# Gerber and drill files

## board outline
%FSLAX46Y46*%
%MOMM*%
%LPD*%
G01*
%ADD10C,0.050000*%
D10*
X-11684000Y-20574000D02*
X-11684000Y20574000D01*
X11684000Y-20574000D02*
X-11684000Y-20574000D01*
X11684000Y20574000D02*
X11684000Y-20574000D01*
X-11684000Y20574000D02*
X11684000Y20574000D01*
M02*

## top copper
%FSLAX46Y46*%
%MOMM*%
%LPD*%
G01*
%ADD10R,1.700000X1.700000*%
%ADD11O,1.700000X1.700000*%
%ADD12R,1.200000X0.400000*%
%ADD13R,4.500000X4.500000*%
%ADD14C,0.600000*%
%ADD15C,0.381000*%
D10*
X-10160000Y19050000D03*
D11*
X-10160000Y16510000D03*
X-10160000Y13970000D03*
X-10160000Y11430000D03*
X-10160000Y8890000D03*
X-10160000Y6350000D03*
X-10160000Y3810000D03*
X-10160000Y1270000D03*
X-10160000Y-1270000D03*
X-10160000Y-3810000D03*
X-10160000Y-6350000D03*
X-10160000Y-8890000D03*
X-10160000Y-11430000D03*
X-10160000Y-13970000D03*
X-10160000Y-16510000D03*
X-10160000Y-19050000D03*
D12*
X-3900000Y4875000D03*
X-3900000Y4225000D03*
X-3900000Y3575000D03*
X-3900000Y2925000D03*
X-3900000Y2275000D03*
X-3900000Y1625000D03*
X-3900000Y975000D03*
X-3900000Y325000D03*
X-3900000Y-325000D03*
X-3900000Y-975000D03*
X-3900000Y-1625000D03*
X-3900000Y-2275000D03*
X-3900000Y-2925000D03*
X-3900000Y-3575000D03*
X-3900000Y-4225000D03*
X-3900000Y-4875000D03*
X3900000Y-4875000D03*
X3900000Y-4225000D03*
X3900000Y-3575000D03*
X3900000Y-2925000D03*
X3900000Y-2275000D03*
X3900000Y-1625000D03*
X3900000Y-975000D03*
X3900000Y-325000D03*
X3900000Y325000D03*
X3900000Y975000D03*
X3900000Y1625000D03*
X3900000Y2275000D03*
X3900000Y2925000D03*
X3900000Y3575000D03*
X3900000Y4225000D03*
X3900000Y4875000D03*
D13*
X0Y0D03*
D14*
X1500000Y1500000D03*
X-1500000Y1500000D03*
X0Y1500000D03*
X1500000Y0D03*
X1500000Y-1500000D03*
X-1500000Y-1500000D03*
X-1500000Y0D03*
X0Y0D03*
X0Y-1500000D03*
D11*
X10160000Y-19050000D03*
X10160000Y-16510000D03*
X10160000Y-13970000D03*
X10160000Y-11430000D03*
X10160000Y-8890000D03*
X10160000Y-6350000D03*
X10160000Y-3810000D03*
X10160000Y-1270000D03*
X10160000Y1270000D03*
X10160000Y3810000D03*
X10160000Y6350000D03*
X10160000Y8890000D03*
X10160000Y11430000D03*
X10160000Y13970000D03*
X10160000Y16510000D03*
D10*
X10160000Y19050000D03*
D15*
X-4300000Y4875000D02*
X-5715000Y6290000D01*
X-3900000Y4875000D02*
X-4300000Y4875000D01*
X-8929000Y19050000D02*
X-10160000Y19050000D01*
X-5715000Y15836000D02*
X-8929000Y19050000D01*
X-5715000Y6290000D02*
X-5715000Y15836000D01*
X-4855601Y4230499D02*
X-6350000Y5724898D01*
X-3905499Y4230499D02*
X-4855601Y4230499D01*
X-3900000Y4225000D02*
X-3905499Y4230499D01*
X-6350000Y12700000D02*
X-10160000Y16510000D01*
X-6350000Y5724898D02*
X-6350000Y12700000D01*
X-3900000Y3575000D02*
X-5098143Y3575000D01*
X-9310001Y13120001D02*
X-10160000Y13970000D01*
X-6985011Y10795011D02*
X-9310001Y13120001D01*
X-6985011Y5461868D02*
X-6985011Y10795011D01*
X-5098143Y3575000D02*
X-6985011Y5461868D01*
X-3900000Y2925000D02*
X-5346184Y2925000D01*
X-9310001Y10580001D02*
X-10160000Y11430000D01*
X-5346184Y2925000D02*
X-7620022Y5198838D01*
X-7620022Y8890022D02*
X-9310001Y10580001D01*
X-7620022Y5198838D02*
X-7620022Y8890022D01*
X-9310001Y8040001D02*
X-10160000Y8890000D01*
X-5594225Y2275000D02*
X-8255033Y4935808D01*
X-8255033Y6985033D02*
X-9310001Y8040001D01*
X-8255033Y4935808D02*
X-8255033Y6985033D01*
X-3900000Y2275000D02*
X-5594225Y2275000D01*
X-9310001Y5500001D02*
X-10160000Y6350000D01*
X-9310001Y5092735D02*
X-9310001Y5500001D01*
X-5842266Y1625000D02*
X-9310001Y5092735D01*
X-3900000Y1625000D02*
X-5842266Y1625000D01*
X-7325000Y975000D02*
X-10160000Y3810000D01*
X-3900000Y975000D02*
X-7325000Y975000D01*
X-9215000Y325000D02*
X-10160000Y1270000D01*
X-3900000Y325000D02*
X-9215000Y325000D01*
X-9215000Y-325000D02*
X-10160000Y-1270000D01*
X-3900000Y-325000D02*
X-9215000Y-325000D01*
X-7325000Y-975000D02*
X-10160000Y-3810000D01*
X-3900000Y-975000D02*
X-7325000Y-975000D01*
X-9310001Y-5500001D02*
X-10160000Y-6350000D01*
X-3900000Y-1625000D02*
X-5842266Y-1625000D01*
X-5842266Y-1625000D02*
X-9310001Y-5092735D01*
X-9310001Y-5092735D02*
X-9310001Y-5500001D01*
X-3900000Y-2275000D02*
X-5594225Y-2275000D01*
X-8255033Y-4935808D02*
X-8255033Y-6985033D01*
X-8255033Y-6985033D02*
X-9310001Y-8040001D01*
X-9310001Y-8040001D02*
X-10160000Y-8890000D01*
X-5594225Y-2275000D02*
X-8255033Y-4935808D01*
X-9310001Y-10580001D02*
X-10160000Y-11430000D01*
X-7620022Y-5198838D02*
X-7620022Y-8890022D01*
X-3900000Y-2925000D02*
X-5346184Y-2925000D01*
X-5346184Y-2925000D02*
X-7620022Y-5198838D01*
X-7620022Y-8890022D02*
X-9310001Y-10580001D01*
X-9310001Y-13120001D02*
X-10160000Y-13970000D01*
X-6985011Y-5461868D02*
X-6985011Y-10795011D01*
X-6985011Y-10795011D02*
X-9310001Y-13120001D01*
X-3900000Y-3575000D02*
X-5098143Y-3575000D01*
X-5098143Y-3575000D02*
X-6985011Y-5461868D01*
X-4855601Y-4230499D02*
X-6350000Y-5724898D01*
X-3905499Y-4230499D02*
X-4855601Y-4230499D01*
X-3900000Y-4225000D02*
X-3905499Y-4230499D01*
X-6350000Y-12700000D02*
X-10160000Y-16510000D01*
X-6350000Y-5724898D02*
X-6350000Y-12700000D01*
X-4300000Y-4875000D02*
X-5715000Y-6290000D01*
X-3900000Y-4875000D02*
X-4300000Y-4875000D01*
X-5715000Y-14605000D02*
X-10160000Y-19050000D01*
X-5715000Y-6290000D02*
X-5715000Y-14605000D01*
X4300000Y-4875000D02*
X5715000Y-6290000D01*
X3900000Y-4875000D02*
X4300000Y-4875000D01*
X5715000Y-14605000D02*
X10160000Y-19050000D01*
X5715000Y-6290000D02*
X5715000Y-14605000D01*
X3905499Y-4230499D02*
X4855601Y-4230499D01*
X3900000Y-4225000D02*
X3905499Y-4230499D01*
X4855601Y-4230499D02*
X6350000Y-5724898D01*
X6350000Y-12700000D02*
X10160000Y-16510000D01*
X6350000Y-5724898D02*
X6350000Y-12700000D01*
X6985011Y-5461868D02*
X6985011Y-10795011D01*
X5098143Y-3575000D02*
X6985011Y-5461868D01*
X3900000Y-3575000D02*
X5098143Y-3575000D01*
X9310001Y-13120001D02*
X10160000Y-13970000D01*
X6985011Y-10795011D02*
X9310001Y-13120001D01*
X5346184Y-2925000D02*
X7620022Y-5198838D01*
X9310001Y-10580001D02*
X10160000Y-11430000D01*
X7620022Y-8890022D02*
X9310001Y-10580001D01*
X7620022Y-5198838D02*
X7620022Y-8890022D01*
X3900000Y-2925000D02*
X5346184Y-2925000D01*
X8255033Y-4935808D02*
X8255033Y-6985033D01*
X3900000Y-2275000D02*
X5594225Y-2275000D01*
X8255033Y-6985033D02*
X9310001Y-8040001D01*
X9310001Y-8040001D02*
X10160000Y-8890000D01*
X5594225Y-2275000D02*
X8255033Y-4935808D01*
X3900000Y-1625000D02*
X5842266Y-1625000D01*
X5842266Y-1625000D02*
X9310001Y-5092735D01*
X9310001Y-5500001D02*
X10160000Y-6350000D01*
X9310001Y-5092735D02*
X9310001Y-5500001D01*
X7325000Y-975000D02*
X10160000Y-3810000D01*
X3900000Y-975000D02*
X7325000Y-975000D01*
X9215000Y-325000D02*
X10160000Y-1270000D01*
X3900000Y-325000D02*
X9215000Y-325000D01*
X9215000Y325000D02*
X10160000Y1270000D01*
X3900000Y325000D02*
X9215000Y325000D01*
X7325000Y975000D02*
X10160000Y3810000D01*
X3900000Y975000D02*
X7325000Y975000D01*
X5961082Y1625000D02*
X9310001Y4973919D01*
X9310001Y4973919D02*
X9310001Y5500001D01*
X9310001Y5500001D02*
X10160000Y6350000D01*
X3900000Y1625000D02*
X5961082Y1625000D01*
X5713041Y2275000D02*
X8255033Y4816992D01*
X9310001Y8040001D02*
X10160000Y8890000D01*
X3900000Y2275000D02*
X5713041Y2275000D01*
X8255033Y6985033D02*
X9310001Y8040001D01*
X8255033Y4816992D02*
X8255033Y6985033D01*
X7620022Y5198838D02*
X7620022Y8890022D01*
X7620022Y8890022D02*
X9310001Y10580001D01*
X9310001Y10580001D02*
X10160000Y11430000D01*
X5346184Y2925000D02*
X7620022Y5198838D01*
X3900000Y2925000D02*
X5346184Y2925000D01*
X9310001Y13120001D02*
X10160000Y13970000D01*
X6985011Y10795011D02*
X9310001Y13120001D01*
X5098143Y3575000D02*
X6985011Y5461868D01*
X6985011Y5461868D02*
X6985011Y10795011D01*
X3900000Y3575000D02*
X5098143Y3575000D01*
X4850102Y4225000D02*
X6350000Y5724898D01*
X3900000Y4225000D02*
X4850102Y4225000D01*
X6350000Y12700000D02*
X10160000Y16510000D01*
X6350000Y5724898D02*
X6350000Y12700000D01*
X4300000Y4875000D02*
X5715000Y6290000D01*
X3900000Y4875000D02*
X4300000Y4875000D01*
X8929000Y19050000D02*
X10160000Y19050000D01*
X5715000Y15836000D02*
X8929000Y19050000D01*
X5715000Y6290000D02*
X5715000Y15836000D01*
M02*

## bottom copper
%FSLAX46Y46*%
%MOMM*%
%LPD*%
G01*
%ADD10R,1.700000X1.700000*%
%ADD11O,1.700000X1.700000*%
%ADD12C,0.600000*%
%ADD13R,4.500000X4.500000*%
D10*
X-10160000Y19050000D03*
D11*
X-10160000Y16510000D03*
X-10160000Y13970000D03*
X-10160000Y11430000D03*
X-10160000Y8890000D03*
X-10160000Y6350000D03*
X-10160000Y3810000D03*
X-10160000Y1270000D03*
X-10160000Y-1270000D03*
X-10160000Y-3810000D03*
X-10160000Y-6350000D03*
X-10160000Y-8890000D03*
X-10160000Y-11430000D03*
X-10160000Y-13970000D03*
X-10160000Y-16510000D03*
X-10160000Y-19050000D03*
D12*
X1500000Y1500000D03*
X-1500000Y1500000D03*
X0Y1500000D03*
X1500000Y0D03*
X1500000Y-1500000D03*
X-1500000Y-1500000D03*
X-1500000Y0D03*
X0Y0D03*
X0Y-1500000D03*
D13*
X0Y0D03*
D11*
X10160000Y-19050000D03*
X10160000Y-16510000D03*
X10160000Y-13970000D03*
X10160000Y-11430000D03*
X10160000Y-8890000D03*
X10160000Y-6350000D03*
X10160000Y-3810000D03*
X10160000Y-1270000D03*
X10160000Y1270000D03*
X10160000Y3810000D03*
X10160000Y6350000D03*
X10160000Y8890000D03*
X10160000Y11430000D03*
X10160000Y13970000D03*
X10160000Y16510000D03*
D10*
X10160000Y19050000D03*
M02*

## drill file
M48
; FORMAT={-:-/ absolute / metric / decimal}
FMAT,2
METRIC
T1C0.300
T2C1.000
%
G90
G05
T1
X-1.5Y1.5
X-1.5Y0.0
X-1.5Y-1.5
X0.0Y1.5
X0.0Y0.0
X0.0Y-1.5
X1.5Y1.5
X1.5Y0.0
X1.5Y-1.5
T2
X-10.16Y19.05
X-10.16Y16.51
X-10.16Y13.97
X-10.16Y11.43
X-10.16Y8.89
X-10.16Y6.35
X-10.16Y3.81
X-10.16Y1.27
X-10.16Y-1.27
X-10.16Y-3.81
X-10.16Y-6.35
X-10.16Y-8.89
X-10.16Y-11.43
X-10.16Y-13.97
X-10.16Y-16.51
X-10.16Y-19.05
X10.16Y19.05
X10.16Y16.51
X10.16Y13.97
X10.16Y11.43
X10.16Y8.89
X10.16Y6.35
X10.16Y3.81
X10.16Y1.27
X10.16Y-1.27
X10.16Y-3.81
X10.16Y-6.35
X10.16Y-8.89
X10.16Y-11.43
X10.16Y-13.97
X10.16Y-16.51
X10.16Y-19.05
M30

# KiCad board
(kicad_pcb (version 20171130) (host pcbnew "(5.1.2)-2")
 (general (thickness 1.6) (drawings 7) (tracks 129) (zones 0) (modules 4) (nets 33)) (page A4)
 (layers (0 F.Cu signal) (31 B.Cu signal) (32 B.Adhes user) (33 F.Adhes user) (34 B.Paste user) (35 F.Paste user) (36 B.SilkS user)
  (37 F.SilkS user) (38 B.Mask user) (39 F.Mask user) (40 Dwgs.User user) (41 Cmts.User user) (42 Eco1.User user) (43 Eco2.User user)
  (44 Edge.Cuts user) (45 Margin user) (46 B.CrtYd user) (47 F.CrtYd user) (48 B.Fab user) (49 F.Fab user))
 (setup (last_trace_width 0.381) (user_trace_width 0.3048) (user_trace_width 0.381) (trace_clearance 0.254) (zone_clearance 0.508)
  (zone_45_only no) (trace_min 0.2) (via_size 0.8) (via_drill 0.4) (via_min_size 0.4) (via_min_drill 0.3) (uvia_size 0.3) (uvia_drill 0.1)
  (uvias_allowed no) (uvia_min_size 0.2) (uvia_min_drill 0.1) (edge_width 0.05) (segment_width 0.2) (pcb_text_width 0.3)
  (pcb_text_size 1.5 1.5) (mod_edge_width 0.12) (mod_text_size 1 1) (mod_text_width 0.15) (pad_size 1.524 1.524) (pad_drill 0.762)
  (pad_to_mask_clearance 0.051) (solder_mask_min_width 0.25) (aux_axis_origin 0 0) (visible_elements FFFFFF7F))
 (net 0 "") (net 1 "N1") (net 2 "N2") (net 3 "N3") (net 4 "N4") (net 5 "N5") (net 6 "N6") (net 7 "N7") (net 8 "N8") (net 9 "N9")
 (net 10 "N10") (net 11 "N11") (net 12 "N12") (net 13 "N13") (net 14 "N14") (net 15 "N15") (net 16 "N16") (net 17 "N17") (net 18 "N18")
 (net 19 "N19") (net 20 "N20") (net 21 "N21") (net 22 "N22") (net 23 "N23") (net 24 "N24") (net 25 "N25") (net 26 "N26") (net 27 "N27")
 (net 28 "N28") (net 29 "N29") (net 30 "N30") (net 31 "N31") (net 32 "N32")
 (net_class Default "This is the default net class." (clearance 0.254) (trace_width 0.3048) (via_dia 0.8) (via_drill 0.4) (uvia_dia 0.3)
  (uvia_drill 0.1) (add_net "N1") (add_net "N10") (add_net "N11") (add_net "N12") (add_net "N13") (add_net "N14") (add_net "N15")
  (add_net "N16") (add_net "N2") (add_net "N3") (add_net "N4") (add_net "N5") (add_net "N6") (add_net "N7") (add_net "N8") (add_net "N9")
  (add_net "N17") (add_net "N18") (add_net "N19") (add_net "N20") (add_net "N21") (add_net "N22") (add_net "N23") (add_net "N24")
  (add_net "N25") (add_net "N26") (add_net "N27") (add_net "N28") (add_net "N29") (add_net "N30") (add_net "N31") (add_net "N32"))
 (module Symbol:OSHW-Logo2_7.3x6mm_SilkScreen (layer F.Cu) (at 0 10.668)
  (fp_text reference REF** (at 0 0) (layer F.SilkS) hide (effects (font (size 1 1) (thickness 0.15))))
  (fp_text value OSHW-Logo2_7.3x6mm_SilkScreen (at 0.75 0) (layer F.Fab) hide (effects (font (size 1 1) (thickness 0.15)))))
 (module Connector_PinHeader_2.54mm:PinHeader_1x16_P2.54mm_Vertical (layer B.Cu) (at -10.16 -19.05 180)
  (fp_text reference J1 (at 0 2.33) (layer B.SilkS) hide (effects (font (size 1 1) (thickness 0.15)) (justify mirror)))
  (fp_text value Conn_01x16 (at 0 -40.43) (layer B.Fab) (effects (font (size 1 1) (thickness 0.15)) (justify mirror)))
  (pad 1 thru_hole rect (at 0 0 180) (size 1.7 1.7) (drill 1) (layers *.Cu *.Mask) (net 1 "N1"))
  (pad 2 thru_hole oval (at 0 -2.54 180) (size 1.7 1.7) (drill 1) (layers *.Cu *.Mask) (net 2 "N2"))
  (pad 3 thru_hole oval (at 0 -5.08 180) (size 1.7 1.7) (drill 1) (layers *.Cu *.Mask) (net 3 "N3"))
  (pad 4 thru_hole oval (at 0 -7.62 180) (size 1.7 1.7) (drill 1) (layers *.Cu *.Mask) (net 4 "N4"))
  (pad 5 thru_hole oval (at 0 -10.16 180) (size 1.7 1.7) (drill 1) (layers *.Cu *.Mask) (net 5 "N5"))
  (pad 6 thru_hole oval (at 0 -12.7 180) (size 1.7 1.7) (drill 1) (layers *.Cu *.Mask) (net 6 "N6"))
  (pad 7 thru_hole oval (at 0 -15.24 180) (size 1.7 1.7) (drill 1) (layers *.Cu *.Mask) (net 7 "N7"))
  (pad 8 thru_hole oval (at 0 -17.78 180) (size 1.7 1.7) (drill 1) (layers *.Cu *.Mask) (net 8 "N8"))
  (pad 9 thru_hole oval (at 0 -20.32 180) (size 1.7 1.7) (drill 1) (layers *.Cu *.Mask) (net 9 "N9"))
  (pad 10 thru_hole oval (at 0 -22.86 180) (size 1.7 1.7) (drill 1) (layers *.Cu *.Mask) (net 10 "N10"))
  (pad 11 thru_hole oval (at 0 -25.4 180) (size 1.7 1.7) (drill 1) (layers *.Cu *.Mask) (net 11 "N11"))
  (pad 12 thru_hole oval (at 0 -27.94 180) (size 1.7 1.7) (drill 1) (layers *.Cu *.Mask) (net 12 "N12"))
  (pad 13 thru_hole oval (at 0 -30.48 180) (size 1.7 1.7) (drill 1) (layers *.Cu *.Mask) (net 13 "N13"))
  (pad 14 thru_hole oval (at 0 -33.02 180) (size 1.7 1.7) (drill 1) (layers *.Cu *.Mask) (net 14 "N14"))
  (pad 15 thru_hole oval (at 0 -35.56 180) (size 1.7 1.7) (drill 1) (layers *.Cu *.Mask) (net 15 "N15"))
  (pad 16 thru_hole oval (at 0 -38.1 180) (size 1.7 1.7) (drill 1) (layers *.Cu *.Mask) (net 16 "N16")))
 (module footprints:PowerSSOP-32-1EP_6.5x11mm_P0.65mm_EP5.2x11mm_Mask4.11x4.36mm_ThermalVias (layer F.Cu) (at 0 0)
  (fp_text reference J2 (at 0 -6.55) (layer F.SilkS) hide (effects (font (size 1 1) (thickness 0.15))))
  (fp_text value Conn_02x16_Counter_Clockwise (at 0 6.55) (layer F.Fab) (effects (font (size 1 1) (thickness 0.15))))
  (pad 1 smd rect (at -3.9 -4.875) (size 1.2 0.4) (layers F.Cu F.Paste F.Mask) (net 1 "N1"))
  (pad 2 smd rect (at -3.9 -4.225) (size 1.2 0.4) (layers F.Cu F.Paste F.Mask) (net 2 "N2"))
  (pad 3 smd rect (at -3.9 -3.575) (size 1.2 0.4) (layers F.Cu F.Paste F.Mask) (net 3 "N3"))
  (pad 4 smd rect (at -3.9 -2.925) (size 1.2 0.4) (layers F.Cu F.Paste F.Mask) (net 4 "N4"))
  (pad 5 smd rect (at -3.9 -2.275) (size 1.2 0.4) (layers F.Cu F.Paste F.Mask) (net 5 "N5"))
  (pad 6 smd rect (at -3.9 -1.625) (size 1.2 0.4) (layers F.Cu F.Paste F.Mask) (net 6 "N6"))
  (pad 7 smd rect (at -3.9 -0.975) (size 1.2 0.4) (layers F.Cu F.Paste F.Mask) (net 7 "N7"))
  (pad 8 smd rect (at -3.9 -0.325) (size 1.2 0.4) (layers F.Cu F.Paste F.Mask) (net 8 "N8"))
  (pad 9 smd rect (at -3.9 0.325) (size 1.2 0.4) (layers F.Cu F.Paste F.Mask) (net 9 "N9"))
  (pad 10 smd rect (at -3.9 0.975) (size 1.2 0.4) (layers F.Cu F.Paste F.Mask) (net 10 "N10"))
  (pad 11 smd rect (at -3.9 1.625) (size 1.2 0.4) (layers F.Cu F.Paste F.Mask) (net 11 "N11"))
  (pad 12 smd rect (at -3.9 2.275) (size 1.2 0.4) (layers F.Cu F.Paste F.Mask) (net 12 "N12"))
  (pad 13 smd rect (at -3.9 2.925) (size 1.2 0.4) (layers F.Cu F.Paste F.Mask) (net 13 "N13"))
  (pad 14 smd rect (at -3.9 3.575) (size 1.2 0.4) (layers F.Cu F.Paste F.Mask) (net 14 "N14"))
  (pad 15 smd rect (at -3.9 4.225) (size 1.2 0.4) (layers F.Cu F.Paste F.Mask) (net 15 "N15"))
  (pad 16 smd rect (at -3.9 4.875) (size 1.2 0.4) (layers F.Cu F.Paste F.Mask) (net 16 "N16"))
  (pad 17 smd rect (at 3.9 4.875) (size 1.2 0.4) (layers F.Cu F.Paste F.Mask) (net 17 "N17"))
  (pad 18 smd rect (at 3.9 4.225) (size 1.2 0.4) (layers F.Cu F.Paste F.Mask) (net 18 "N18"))
  (pad 19 smd rect (at 3.9 3.575) (size 1.2 0.4) (layers F.Cu F.Paste F.Mask) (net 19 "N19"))
  (pad 20 smd rect (at 3.9 2.925) (size 1.2 0.4) (layers F.Cu F.Paste F.Mask) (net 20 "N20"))
  (pad 21 smd rect (at 3.9 2.275) (size 1.2 0.4) (layers F.Cu F.Paste F.Mask) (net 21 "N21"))
  (pad 22 smd rect (at 3.9 1.625) (size 1.2 0.4) (layers F.Cu F.Paste F.Mask) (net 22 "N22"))
  (pad 23 smd rect (at 3.9 0.975) (size 1.2 0.4) (layers F.Cu F.Paste F.Mask) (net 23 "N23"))
  (pad 24 smd rect (at 3.9 0.325) (size 1.2 0.4) (layers F.Cu F.Paste F.Mask) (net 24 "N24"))
  (pad 25 smd rect (at 3.9 -0.325) (size 1.2 0.4) (layers F.Cu F.Paste F.Mask) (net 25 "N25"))
  (pad 26 smd rect (at 3.9 -0.975) (size 1.2 0.4) (layers F.Cu F.Paste F.Mask) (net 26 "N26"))
  (pad 27 smd rect (at 3.9 -1.625) (size 1.2 0.4) (layers F.Cu F.Paste F.Mask) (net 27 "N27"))
  (pad 28 smd rect (at 3.9 -2.275) (size 1.2 0.4) (layers F.Cu F.Paste F.Mask) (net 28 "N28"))
  (pad 29 smd rect (at 3.9 -2.925) (size 1.2 0.4) (layers F.Cu F.Paste F.Mask) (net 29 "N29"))
  (pad 30 smd rect (at 3.9 -3.575) (size 1.2 0.4) (layers F.Cu F.Paste F.Mask) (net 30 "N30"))
  (pad 31 smd rect (at 3.9 -4.225) (size 1.2 0.4) (layers F.Cu F.Paste F.Mask) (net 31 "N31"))
  (pad 32 smd rect (at 3.9 -4.875) (size 1.2 0.4) (layers F.Cu F.Paste F.Mask) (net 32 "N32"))
  (pad 33 smd rect (at 0 0) (size 4.5 4.5) (layers F.Cu)) (pad "" smd rect (at 0 0) (size 4.11 4.36) (layers F.Mask))
  (pad 33 thru_hole circle (at 1.5 -1.5) (size 0.6 0.6) (drill 0.3) (layers *.Cu))
  (pad 33 thru_hole circle (at -1.5 -1.5) (size 0.6 0.6) (drill 0.3) (layers *.Cu))
  (pad 33 thru_hole circle (at 0 -1.5) (size 0.6 0.6) (drill 0.3) (layers *.Cu))
  (pad 33 thru_hole circle (at 1.5 0) (size 0.6 0.6) (drill 0.3) (layers *.Cu))
  (pad 33 thru_hole circle (at 1.5 1.5) (size 0.6 0.6) (drill 0.3) (layers *.Cu))
  (pad 33 thru_hole circle (at -1.5 1.5) (size 0.6 0.6) (drill 0.3) (layers *.Cu))
  (pad 33 thru_hole circle (at -1.5 0) (size 0.6 0.6) (drill 0.3) (layers *.Cu))
  (pad 33 thru_hole circle (at 0 0) (size 0.6 0.6) (drill 0.3) (layers *.Cu))
  (pad 33 thru_hole circle (at 0 1.5) (size 0.6 0.6) (drill 0.3) (layers *.Cu)) (pad "" smd rect (at 0 -0.65) (size 1.2 1) (layers F.Paste))
  (pad "" smd rect (at 0 0.65) (size 1.2 1) (layers F.Paste))
  (pad "" smd rect (at 0 1.725) (size 1.2 0.55) (layers F.Paste))
  (pad "" smd rect (at 0 -1.725) (size 1.2 0.55) (layers F.Paste))
  (pad "" smd rect (at -1.365 -0.65) (size 0.93 1) (layers F.Paste))
  (pad "" smd rect (at -1.365 0.65) (size 0.93 1) (layers F.Paste))
  (pad "" smd rect (at 1.365 0.65) (size 0.93 1) (layers F.Paste))
  (pad "" smd rect (at 1.365 -0.65) (size 0.93 1) (layers F.Paste))
  (pad "" smd rect (at 1.365 -1.725) (size 0.93 0.55) (layers F.Paste))
  (pad "" smd rect (at 1.365 1.725) (size 0.93 0.55) (layers F.Paste))
  (pad "" smd rect (at -1.365 1.725) (size 0.93 0.55) (layers F.Paste))
  (pad "" smd rect (at -1.365 -1.725) (size 0.93 0.55) (layers F.Paste)) (pad 33 smd rect (at 0 0) (size 4.5 4.5) (layers B.Cu))
  (pad "" smd rect (at 0 0) (size 4.11 4.36) (layers B.Mask)))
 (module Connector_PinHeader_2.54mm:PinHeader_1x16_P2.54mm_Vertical (layer B.Cu) (at 10.16 -19.05 180)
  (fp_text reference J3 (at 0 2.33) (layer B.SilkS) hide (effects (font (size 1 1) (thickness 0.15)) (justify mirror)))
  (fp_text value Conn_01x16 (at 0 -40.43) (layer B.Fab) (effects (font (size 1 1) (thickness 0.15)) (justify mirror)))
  (pad 16 thru_hole oval (at 0 -38.1 180) (size 1.7 1.7) (drill 1) (layers *.Cu *.Mask) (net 17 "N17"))
  (pad 15 thru_hole oval (at 0 -35.56 180) (size 1.7 1.7) (drill 1) (layers *.Cu *.Mask) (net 18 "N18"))
  (pad 14 thru_hole oval (at 0 -33.02 180) (size 1.7 1.7) (drill 1) (layers *.Cu *.Mask) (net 19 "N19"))
  (pad 13 thru_hole oval (at 0 -30.48 180) (size 1.7 1.7) (drill 1) (layers *.Cu *.Mask) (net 20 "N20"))
  (pad 12 thru_hole oval (at 0 -27.94 180) (size 1.7 1.7) (drill 1) (layers *.Cu *.Mask) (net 21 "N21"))
  (pad 11 thru_hole oval (at 0 -25.4 180) (size 1.7 1.7) (drill 1) (layers *.Cu *.Mask) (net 22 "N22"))
  (pad 10 thru_hole oval (at 0 -22.86 180) (size 1.7 1.7) (drill 1) (layers *.Cu *.Mask) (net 23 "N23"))
  (pad 9 thru_hole oval (at 0 -20.32 180) (size 1.7 1.7) (drill 1) (layers *.Cu *.Mask) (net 24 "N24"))
  (pad 8 thru_hole oval (at 0 -17.78 180) (size 1.7 1.7) (drill 1) (layers *.Cu *.Mask) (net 25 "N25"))
  (pad 7 thru_hole oval (at 0 -15.24 180) (size 1.7 1.7) (drill 1) (layers *.Cu *.Mask) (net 26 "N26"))
  (pad 6 thru_hole oval (at 0 -12.7 180) (size 1.7 1.7) (drill 1) (layers *.Cu *.Mask) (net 27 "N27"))
  (pad 5 thru_hole oval (at 0 -10.16 180) (size 1.7 1.7) (drill 1) (layers *.Cu *.Mask) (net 28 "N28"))
  (pad 4 thru_hole oval (at 0 -7.62 180) (size 1.7 1.7) (drill 1) (layers *.Cu *.Mask) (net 29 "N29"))
  (pad 3 thru_hole oval (at 0 -5.08 180) (size 1.7 1.7) (drill 1) (layers *.Cu *.Mask) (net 30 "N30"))
  (pad 2 thru_hole oval (at 0 -2.54 180) (size 1.7 1.7) (drill 1) (layers *.Cu *.Mask) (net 31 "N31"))
  (pad 1 thru_hole rect (at 0 0 180) (size 1.7 1.7) (drill 1) (layers *.Cu *.Mask) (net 32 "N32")))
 (gr_line (start -11.684 20.574) (end -11.684 -20.574) (layer Edge.Cuts) (width 0.05))
 (gr_line (start 11.684 20.574) (end -11.684 20.574) (layer Edge.Cuts) (width 0.05))
 (gr_line (start 11.684 -20.574) (end 11.684 20.574) (layer Edge.Cuts) (width 0.05))
 (gr_line (start -11.684 -20.574) (end 11.684 -20.574) (layer Edge.Cuts) (width 0.05))
 (segment (start -4.3 -4.875) (end -5.715 -6.29) (width 0.381) (layer F.Cu) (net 1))
 (segment (start -3.9 -4.875) (end -4.3 -4.875) (width 0.381) (layer F.Cu) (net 1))
 (segment (start -8.929 -19.05) (end -10.16 -19.05) (width 0.381) (layer F.Cu) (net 1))
 (segment (start -5.715 -15.836) (end -8.929 -19.05) (width 0.381) (layer F.Cu) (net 1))
 (segment (start -5.715 -6.29) (end -5.715 -15.836) (width 0.381) (layer F.Cu) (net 1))
 (segment (start -4.855601 -4.230499) (end -6.35 -5.724898) (width 0.381) (layer F.Cu) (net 2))
 (segment (start -3.905499 -4.230499) (end -4.855601 -4.230499) (width 0.381) (layer F.Cu) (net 2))
 (segment (start -3.9 -4.225) (end -3.905499 -4.230499) (width 0.381) (layer F.Cu) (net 2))
 (segment (start -6.35 -12.7) (end -10.16 -16.51) (width 0.381) (layer F.Cu) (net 2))
 (segment (start -6.35 -5.724898) (end -6.35 -12.7) (width 0.381) (layer F.Cu) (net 2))
 (segment (start -3.9 -3.575) (end -5.098143 -3.575) (width 0.381) (layer F.Cu) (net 3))
 (segment (start -9.310001 -13.120001) (end -10.16 -13.97) (width 0.381) (layer F.Cu) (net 3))
 (segment (start -6.985011 -10.795011) (end -9.310001 -13.120001) (width 0.381) (layer F.Cu) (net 3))
 (segment (start -6.985011 -5.461868) (end -6.985011 -10.795011) (width 0.381) (layer F.Cu) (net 3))
 (segment (start -5.098143 -3.575) (end -6.985011 -5.461868) (width 0.381) (layer F.Cu) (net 3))
 (segment (start -3.9 -2.925) (end -5.346184 -2.925) (width 0.381) (layer F.Cu) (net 4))
 (segment (start -9.310001 -10.580001) (end -10.16 -11.43) (width 0.381) (layer F.Cu) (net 4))
 (segment (start -5.346184 -2.925) (end -7.620022 -5.198838) (width 0.381) (layer F.Cu) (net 4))
 (segment (start -7.620022 -8.890022) (end -9.310001 -10.580001) (width 0.381) (layer F.Cu) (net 4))
 (segment (start -7.620022 -5.198838) (end -7.620022 -8.890022) (width 0.381) (layer F.Cu) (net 4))
 (segment (start -9.310001 -8.040001) (end -10.16 -8.89) (width 0.381) (layer F.Cu) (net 5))
 (segment (start -5.594225 -2.275) (end -8.255033 -4.935808) (width 0.381) (layer F.Cu) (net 5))
 (segment (start -8.255033 -6.985033) (end -9.310001 -8.040001) (width 0.381) (layer F.Cu) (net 5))
 (segment (start -8.255033 -4.935808) (end -8.255033 -6.985033) (width 0.381) (layer F.Cu) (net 5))
 (segment (start -3.9 -2.275) (end -5.594225 -2.275) (width 0.381) (layer F.Cu) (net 5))
 (segment (start -9.310001 -5.500001) (end -10.16 -6.35) (width 0.381) (layer F.Cu) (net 6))
 (segment (start -9.310001 -5.092735) (end -9.310001 -5.500001) (width 0.381) (layer F.Cu) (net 6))
 (segment (start -5.842266 -1.625) (end -9.310001 -5.092735) (width 0.381) (layer F.Cu) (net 6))
 (segment (start -3.9 -1.625) (end -5.842266 -1.625) (width 0.381) (layer F.Cu) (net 6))
 (segment (start -7.325 -0.975) (end -10.16 -3.81) (width 0.381) (layer F.Cu) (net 7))
 (segment (start -3.9 -0.975) (end -7.325 -0.975) (width 0.381) (layer F.Cu) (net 7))
 (segment (start -9.215 -0.325) (end -10.16 -1.27) (width 0.381) (layer F.Cu) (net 8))
 (segment (start -3.9 -0.325) (end -9.215 -0.325) (width 0.381) (layer F.Cu) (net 8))
 (segment (start -9.215 0.325) (end -10.16 1.27) (width 0.381) (layer F.Cu) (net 9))
 (segment (start -3.9 0.325) (end -9.215 0.325) (width 0.381) (layer F.Cu) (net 9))
 (segment (start -7.325 0.975) (end -10.16 3.81) (width 0.381) (layer F.Cu) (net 10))
 (segment (start -3.9 0.975) (end -7.325 0.975) (width 0.381) (layer F.Cu) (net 10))
 (segment (start -9.310001 5.500001) (end -10.16 6.35) (width 0.381) (layer F.Cu) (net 11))
 (segment (start -3.9 1.625) (end -5.842266 1.625) (width 0.381) (layer F.Cu) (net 11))
 (segment (start -5.842266 1.625) (end -9.310001 5.092735) (width 0.381) (layer F.Cu) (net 11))
 (segment (start -9.310001 5.092735) (end -9.310001 5.500001) (width 0.381) (layer F.Cu) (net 11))
 (segment (start -3.9 2.275) (end -5.594225 2.275) (width 0.381) (layer F.Cu) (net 12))
 (segment (start -8.255033 4.935808) (end -8.255033 6.985033) (width 0.381) (layer F.Cu) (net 12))
 (segment (start -8.255033 6.985033) (end -9.310001 8.040001) (width 0.381) (layer F.Cu) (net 12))
 (segment (start -9.310001 8.040001) (end -10.16 8.89) (width 0.381) (layer F.Cu) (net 12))
 (segment (start -5.594225 2.275) (end -8.255033 4.935808) (width 0.381) (layer F.Cu) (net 12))
 (segment (start -9.310001 10.580001) (end -10.16 11.43) (width 0.381) (layer F.Cu) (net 13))
 (segment (start -7.620022 5.198838) (end -7.620022 8.890022) (width 0.381) (layer F.Cu) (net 13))
 (segment (start -3.9 2.925) (end -5.346184 2.925) (width 0.381) (layer F.Cu) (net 13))
 (segment (start -5.346184 2.925) (end -7.620022 5.198838) (width 0.381) (layer F.Cu) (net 13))
 (segment (start -7.620022 8.890022) (end -9.310001 10.580001) (width 0.381) (layer F.Cu) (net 13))
 (segment (start -9.310001 13.120001) (end -10.16 13.97) (width 0.381) (layer F.Cu) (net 14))
 (segment (start -6.985011 5.461868) (end -6.985011 10.795011) (width 0.381) (layer F.Cu) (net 14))
 (segment (start -6.985011 10.795011) (end -9.310001 13.120001) (width 0.381) (layer F.Cu) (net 14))
 (segment (start -3.9 3.575) (end -5.098143 3.575) (width 0.381) (layer F.Cu) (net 14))
 (segment (start -5.098143 3.575) (end -6.985011 5.461868) (width 0.381) (layer F.Cu) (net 14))
 (segment (start -4.855601 4.230499) (end -6.35 5.724898) (width 0.381) (layer F.Cu) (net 15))
 (segment (start -3.905499 4.230499) (end -4.855601 4.230499) (width 0.381) (layer F.Cu) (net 15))
 (segment (start -3.9 4.225) (end -3.905499 4.230499) (width 0.381) (layer F.Cu) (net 15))
 (segment (start -6.35 12.7) (end -10.16 16.51) (width 0.381) (layer F.Cu) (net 15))
 (segment (start -6.35 5.724898) (end -6.35 12.7) (width 0.381) (layer F.Cu) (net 15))
 (segment (start -4.3 4.875) (end -5.715 6.29) (width 0.381) (layer F.Cu) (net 16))
 (segment (start -3.9 4.875) (end -4.3 4.875) (width 0.381) (layer F.Cu) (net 16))
 (segment (start -5.715 14.605) (end -10.16 19.05) (width 0.381) (layer F.Cu) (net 16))
 (segment (start -5.715 6.29) (end -5.715 14.605) (width 0.381) (layer F.Cu) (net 16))
 (segment (start 4.3 4.875) (end 5.715 6.29) (width 0.381) (layer F.Cu) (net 17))
 (segment (start 3.9 4.875) (end 4.3 4.875) (width 0.381) (layer F.Cu) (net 17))
 (segment (start 5.715 14.605) (end 10.16 19.05) (width 0.381) (layer F.Cu) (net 17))
 (segment (start 5.715 6.29) (end 5.715 14.605) (width 0.381) (layer F.Cu) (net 17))
 (segment (start 3.905499 4.230499) (end 4.855601 4.230499) (width 0.381) (layer F.Cu) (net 18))
 (segment (start 3.9 4.225) (end 3.905499 4.230499) (width 0.381) (layer F.Cu) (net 18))
 (segment (start 4.855601 4.230499) (end 6.35 5.724898) (width 0.381) (layer F.Cu) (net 18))
 (segment (start 6.35 12.7) (end 10.16 16.51) (width 0.381) (layer F.Cu) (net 18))
 (segment (start 6.35 5.724898) (end 6.35 12.7) (width 0.381) (layer F.Cu) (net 18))
 (segment (start 6.985011 5.461868) (end 6.985011 10.795011) (width 0.381) (layer F.Cu) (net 19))
 (segment (start 5.098143 3.575) (end 6.985011 5.461868) (width 0.381) (layer F.Cu) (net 19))
 (segment (start 3.9 3.575) (end 5.098143 3.575) (width 0.381) (layer F.Cu) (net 19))
 (segment (start 9.310001 13.120001) (end 10.16 13.97) (width 0.381) (layer F.Cu) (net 19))
 (segment (start 6.985011 10.795011) (end 9.310001 13.120001) (width 0.381) (layer F.Cu) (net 19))
 (segment (start 5.346184 2.925) (end 7.620022 5.198838) (width 0.381) (layer F.Cu) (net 20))
 (segment (start 9.310001 10.580001) (end 10.16 11.43) (width 0.381) (layer F.Cu) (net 20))
 (segment (start 7.620022 8.890022) (end 9.310001 10.580001) (width 0.381) (layer F.Cu) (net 20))
 (segment (start 7.620022 5.198838) (end 7.620022 8.890022) (width 0.381) (layer F.Cu) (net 20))
 (segment (start 3.9 2.925) (end 5.346184 2.925) (width 0.381) (layer F.Cu) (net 20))
 (segment (start 8.255033 4.935808) (end 8.255033 6.985033) (width 0.381) (layer F.Cu) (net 21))
 (segment (start 3.9 2.275) (end 5.594225 2.275) (width 0.381) (layer F.Cu) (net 21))
 (segment (start 8.255033 6.985033) (end 9.310001 8.040001) (width 0.381) (layer F.Cu) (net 21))
 (segment (start 9.310001 8.040001) (end 10.16 8.89) (width 0.381) (layer F.Cu) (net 21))
 (segment (start 5.594225 2.275) (end 8.255033 4.935808) (width 0.381) (layer F.Cu) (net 21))
 (segment (start 3.9 1.625) (end 5.842266 1.625) (width 0.381) (layer F.Cu) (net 22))
 (segment (start 5.842266 1.625) (end 9.310001 5.092735) (width 0.381) (layer F.Cu) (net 22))
 (segment (start 9.310001 5.500001) (end 10.16 6.35) (width 0.381) (layer F.Cu) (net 22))
 (segment (start 9.310001 5.092735) (end 9.310001 5.500001) (width 0.381) (layer F.Cu) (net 22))
 (segment (start 7.325 0.975) (end 10.16 3.81) (width 0.381) (layer F.Cu) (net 23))
 (segment (start 3.9 0.975) (end 7.325 0.975) (width 0.381) (layer F.Cu) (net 23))
 (segment (start 9.215 0.325) (end 10.16 1.27) (width 0.381) (layer F.Cu) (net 24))
 (segment (start 3.9 0.325) (end 9.215 0.325) (width 0.381) (layer F.Cu) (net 24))
 (segment (start 9.215 -0.325) (end 10.16 -1.27) (width 0.381) (layer F.Cu) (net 25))
 (segment (start 3.9 -0.325) (end 9.215 -0.325) (width 0.381) (layer F.Cu) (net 25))
 (segment (start 7.325 -0.975) (end 10.16 -3.81) (width 0.381) (layer F.Cu) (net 26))
 (segment (start 3.9 -0.975) (end 7.325 -0.975) (width 0.381) (layer F.Cu) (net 26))
 (segment (start 5.961082 -1.625) (end 9.310001 -4.973919) (width 0.381) (layer F.Cu) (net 27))
 (segment (start 9.310001 -4.973919) (end 9.310001 -5.500001) (width 0.381) (layer F.Cu) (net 27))
 (segment (start 9.310001 -5.500001) (end 10.16 -6.35) (width 0.381) (layer F.Cu) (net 27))
 (segment (start 3.9 -1.625) (end 5.961082 -1.625) (width 0.381) (layer F.Cu) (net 27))
 (segment (start 5.713041 -2.275) (end 8.255033 -4.816992) (width 0.381) (layer F.Cu) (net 28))
 (segment (start 9.310001 -8.040001) (end 10.16 -8.89) (width 0.381) (layer F.Cu) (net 28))
 (segment (start 3.9 -2.275) (end 5.713041 -2.275) (width 0.381) (layer F.Cu) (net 28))
 (segment (start 8.255033 -6.985033) (end 9.310001 -8.040001) (width 0.381) (layer F.Cu) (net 28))
 (segment (start 8.255033 -4.816992) (end 8.255033 -6.985033) (width 0.381) (layer F.Cu) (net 28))
 (segment (start 7.620022 -5.198838) (end 7.620022 -8.890022) (width 0.381) (layer F.Cu) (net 29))
 (segment (start 7.620022 -8.890022) (end 9.310001 -10.580001) (width 0.381) (layer F.Cu) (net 29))
 (segment (start 9.310001 -10.580001) (end 10.16 -11.43) (width 0.381) (layer F.Cu) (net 29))
 (segment (start 5.346184 -2.925) (end 7.620022 -5.198838) (width 0.381) (layer F.Cu) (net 29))
 (segment (start 3.9 -2.925) (end 5.346184 -2.925) (width 0.381) (layer F.Cu) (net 29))
 (segment (start 9.310001 -13.120001) (end 10.16 -13.97) (width 0.381) (layer F.Cu) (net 30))
 (segment (start 6.985011 -10.795011) (end 9.310001 -13.120001) (width 0.381) (layer F.Cu) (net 30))
 (segment (start 5.098143 -3.575) (end 6.985011 -5.461868) (width 0.381) (layer F.Cu) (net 30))
 (segment (start 6.985011 -5.461868) (end 6.985011 -10.795011) (width 0.381) (layer F.Cu) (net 30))
 (segment (start 3.9 -3.575) (end 5.098143 -3.575) (width 0.381) (layer F.Cu) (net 30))
 (segment (start 4.850102 -4.225) (end 6.35 -5.724898) (width 0.381) (layer F.Cu) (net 31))
 (segment (start 3.9 -4.225) (end 4.850102 -4.225) (width 0.381) (layer F.Cu) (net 31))
 (segment (start 6.35 -12.7) (end 10.16 -16.51) (width 0.381) (layer F.Cu) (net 31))
 (segment (start 6.35 -5.724898) (end 6.35 -12.7) (width 0.381) (layer F.Cu) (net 31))
 (segment (start 4.3 -4.875) (end 5.715 -6.29) (width 0.381) (layer F.Cu) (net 32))
 (segment (start 3.9 -4.875) (end 4.3 -4.875) (width 0.381) (layer F.Cu) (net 32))
 (segment (start 8.929 -19.05) (end 10.16 -19.05) (width 0.381) (layer F.Cu) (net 32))
 (segment (start 5.715 -15.836) (end 8.929 -19.05) (width 0.381) (layer F.Cu) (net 32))
 (segment (start 5.715 -6.29) (end 5.715 -15.836) (width 0.381) (layer F.Cu) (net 32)))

